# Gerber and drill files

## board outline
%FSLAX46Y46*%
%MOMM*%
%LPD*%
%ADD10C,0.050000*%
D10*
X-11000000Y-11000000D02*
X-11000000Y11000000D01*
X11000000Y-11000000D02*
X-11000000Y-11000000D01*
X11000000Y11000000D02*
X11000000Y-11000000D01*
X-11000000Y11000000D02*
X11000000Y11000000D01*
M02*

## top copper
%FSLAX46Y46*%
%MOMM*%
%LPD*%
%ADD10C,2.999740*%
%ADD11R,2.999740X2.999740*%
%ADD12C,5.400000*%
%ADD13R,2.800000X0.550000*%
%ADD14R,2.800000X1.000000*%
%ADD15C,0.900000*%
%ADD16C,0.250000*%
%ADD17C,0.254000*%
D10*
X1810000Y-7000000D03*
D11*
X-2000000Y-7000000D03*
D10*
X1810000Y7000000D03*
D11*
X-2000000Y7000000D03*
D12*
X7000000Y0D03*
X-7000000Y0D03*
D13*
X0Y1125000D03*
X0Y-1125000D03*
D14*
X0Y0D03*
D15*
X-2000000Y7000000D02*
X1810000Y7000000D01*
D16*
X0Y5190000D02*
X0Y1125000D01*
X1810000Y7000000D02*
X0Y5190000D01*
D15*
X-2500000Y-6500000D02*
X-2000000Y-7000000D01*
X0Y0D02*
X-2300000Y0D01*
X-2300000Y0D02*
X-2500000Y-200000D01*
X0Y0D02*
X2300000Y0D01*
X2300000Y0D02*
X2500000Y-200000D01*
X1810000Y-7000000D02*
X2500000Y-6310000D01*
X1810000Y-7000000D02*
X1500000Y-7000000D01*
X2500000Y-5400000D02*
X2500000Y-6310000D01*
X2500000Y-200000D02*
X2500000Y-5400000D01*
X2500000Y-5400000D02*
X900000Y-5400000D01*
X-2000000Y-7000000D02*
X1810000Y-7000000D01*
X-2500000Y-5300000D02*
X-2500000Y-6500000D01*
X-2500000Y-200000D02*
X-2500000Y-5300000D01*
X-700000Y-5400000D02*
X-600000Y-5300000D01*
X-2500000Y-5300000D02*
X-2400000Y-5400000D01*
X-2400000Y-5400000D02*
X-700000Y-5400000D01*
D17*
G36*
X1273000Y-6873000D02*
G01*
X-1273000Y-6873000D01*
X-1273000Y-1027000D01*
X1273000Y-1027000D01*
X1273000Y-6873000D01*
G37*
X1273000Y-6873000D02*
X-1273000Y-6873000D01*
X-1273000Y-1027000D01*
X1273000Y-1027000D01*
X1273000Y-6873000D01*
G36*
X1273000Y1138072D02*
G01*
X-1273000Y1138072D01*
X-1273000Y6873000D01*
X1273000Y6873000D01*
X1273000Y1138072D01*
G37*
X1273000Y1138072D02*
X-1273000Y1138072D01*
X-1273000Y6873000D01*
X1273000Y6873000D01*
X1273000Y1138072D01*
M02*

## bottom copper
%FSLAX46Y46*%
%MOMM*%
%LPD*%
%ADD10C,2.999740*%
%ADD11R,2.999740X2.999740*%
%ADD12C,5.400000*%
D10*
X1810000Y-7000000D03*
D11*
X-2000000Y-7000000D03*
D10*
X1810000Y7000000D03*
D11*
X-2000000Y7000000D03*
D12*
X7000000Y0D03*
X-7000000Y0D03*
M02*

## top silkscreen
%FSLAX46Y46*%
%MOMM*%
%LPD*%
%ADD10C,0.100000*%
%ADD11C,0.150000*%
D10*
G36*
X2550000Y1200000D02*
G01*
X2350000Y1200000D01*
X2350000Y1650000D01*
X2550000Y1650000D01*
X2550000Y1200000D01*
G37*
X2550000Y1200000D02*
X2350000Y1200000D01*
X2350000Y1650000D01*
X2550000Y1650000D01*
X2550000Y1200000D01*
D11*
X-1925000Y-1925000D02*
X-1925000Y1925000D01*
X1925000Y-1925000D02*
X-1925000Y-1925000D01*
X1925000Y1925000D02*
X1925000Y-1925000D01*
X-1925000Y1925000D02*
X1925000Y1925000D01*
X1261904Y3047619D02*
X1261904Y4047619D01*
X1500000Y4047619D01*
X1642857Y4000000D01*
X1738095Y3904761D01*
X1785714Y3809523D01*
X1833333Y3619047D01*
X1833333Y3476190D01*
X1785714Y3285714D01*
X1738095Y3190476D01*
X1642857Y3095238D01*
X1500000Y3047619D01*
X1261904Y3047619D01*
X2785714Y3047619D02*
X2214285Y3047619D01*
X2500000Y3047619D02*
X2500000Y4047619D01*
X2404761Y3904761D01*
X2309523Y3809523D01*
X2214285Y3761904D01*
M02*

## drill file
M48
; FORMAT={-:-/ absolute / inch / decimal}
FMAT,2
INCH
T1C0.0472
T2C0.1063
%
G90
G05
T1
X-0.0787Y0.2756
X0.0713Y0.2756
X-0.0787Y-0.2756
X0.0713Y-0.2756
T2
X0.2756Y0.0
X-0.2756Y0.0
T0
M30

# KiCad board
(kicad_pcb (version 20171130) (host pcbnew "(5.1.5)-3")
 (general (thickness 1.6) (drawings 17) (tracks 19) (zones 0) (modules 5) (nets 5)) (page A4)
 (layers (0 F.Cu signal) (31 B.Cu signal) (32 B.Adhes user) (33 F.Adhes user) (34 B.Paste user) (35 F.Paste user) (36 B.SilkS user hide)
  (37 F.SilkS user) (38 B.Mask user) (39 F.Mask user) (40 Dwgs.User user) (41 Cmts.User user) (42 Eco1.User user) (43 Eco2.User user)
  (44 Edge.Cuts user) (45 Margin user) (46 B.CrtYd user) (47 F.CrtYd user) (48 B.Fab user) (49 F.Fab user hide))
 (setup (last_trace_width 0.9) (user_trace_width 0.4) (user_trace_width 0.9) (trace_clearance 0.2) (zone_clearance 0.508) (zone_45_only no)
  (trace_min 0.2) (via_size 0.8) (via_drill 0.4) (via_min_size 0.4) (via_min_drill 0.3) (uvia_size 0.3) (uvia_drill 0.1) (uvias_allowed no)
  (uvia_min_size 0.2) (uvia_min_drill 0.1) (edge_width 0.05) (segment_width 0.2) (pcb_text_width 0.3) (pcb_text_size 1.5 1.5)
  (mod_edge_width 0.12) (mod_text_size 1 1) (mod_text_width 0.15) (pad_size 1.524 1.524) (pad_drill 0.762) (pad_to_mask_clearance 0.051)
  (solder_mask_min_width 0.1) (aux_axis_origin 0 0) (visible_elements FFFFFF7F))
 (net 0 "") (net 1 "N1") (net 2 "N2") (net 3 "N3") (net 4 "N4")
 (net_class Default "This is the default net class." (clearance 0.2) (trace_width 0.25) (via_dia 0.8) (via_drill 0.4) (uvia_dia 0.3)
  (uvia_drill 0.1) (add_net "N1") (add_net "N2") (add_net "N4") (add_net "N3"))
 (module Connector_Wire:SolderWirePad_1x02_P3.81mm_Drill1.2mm (layer F.Cu) (at -2 7)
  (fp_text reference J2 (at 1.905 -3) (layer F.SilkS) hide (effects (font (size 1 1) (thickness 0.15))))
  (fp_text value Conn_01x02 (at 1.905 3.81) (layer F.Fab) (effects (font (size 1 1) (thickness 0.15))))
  (pad 2 thru_hole circle (at 3.81 0) (size 2.99974 2.99974) (drill 1.19888) (layers *.Cu *.Mask) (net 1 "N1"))
  (pad 1 thru_hole rect (at 0 0) (size 2.99974 2.99974) (drill 1.19888) (layers *.Cu *.Mask) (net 1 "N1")))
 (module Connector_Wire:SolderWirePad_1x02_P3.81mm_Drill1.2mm (layer F.Cu) (at -2 -7)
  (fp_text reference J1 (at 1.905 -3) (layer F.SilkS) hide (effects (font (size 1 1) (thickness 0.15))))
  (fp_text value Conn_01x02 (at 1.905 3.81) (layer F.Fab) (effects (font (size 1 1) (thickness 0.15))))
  (pad 2 thru_hole circle (at 3.81 0) (size 2.99974 2.99974) (drill 1.19888) (layers *.Cu *.Mask) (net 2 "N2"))
  (pad 1 thru_hole rect (at 0 0) (size 2.99974 2.99974) (drill 1.19888) (layers *.Cu *.Mask) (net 2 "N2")))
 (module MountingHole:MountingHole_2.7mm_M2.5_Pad (layer F.Cu) (at 7 0)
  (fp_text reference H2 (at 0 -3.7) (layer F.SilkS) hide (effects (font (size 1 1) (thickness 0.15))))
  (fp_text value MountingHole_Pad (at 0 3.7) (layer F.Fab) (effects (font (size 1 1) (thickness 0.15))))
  (pad 1 thru_hole circle (at 0 0) (size 5.4 5.4) (drill 2.7) (layers *.Cu *.Mask) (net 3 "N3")))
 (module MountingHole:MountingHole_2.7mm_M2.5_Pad (layer F.Cu) (at -7 0)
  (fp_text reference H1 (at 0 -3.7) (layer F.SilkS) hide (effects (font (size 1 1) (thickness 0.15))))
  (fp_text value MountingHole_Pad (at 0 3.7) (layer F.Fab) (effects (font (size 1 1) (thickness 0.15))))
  (pad 1 thru_hole circle (at 0 0) (size 5.4 5.4) (drill 2.7) (layers *.Cu *.Mask) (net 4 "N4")))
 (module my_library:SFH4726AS (layer F.Cu) (at 0 0)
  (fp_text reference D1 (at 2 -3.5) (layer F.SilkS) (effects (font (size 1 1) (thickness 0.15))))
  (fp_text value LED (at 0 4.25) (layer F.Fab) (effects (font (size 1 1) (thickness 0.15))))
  (fp_poly (pts (xy 2.55 -1.2) (xy 2.35 -1.2) (xy 2.35 -1.65) (xy 2.55 -1.65)) (layer F.SilkS) (width 0.1))
  (fp_line (start -1.925 1.925) (end -1.925 -1.925) (layer F.SilkS) (width 0.15))
  (fp_line (start 1.925 1.925) (end -1.925 1.925) (layer F.SilkS) (width 0.15))
  (fp_line (start 1.925 -1.925) (end 1.925 1.925) (layer F.SilkS) (width 0.15))
  (fp_line (start -1.925 -1.925) (end 1.925 -1.925) (layer F.SilkS) (width 0.15))
  (pad 2 smd rect (at 0 -1.125) (size 2.8 0.55) (layers F.Cu F.Paste F.Mask) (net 2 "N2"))
  (pad 1 smd rect (at 0 1.125) (size 2.8 0.55) (layers F.Cu F.Paste F.Mask) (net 1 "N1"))
  (pad 1 smd rect (at 0 0) (size 2.8 1) (layers F.Cu F.Mask) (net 1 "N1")))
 (gr_line (start -11 11) (end -11 -11) (layer Edge.Cuts) (width 0.05))
 (gr_line (start 11 11) (end -11 11) (layer Edge.Cuts) (width 0.05))
 (gr_line (start 11 -11) (end 11 11) (layer Edge.Cuts) (width 0.05))
 (gr_line (start -11 -11) (end 11 -11) (layer Edge.Cuts) (width 0.05))
 (segment (start -2 -7) (end 1.81 -7) (width 0.9) (layer F.Cu) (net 2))
 (segment (start 0 -5.19) (end 0 -1.125) (width 0.25) (layer F.Cu) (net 2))
 (segment (start 1.81 -7) (end 0 -5.19) (width 0.25) (layer F.Cu) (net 2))
 (segment (start -2.5 6.5) (end -2 7) (width 0.9) (layer F.Cu) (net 1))
 (segment (start 0 0) (end -2.3 0) (width 0.9) (layer F.Cu) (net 1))
 (segment (start -2.3 0) (end -2.5 0.2) (width 0.9) (layer F.Cu) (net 1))
 (segment (start 0 0) (end 2.3 0) (width 0.9) (layer F.Cu) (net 1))
 (segment (start 2.3 0) (end 2.5 0.2) (width 0.9) (layer F.Cu) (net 1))
 (segment (start 1.81 7) (end 2.5 6.31) (width 0.9) (layer F.Cu) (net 1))
 (segment (start 1.81 7) (end 1.5 7) (width 0.9) (layer F.Cu) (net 1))
 (segment (start 2.5 5.4) (end 2.5 6.31) (width 0.9) (layer F.Cu) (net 1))
 (segment (start 2.5 0.2) (end 2.5 5.4) (width 0.9) (layer F.Cu) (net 1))
 (segment (start 2.5 5.4) (end 0.9 5.4) (width 0.9) (layer F.Cu) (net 1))
 (segment (start -2 7) (end 1.81 7) (width 0.9) (layer F.Cu) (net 1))
 (segment (start -2.5 5.3) (end -2.5 6.5) (width 0.9) (layer F.Cu) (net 1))
 (segment (start -2.5 0.2) (end -2.5 5.3) (width 0.9) (layer F.Cu) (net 1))
 (segment (start -0.7 5.4) (end -0.6 5.3) (width 0.9) (layer F.Cu) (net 1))
 (segment (start -2.5 5.3) (end -2.4 5.4) (width 0.9) (layer F.Cu) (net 1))
 (segment (start -2.4 5.4) (end -0.7 5.4) (width 0.9) (layer F.Cu) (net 1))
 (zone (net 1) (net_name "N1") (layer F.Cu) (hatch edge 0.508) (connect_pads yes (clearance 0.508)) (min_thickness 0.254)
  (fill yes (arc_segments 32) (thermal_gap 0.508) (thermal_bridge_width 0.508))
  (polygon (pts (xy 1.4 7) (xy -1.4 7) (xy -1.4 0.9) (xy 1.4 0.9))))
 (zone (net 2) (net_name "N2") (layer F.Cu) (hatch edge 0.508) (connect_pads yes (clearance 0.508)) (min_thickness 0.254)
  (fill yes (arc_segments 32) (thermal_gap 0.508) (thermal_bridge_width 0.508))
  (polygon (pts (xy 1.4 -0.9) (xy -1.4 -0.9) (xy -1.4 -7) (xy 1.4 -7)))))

